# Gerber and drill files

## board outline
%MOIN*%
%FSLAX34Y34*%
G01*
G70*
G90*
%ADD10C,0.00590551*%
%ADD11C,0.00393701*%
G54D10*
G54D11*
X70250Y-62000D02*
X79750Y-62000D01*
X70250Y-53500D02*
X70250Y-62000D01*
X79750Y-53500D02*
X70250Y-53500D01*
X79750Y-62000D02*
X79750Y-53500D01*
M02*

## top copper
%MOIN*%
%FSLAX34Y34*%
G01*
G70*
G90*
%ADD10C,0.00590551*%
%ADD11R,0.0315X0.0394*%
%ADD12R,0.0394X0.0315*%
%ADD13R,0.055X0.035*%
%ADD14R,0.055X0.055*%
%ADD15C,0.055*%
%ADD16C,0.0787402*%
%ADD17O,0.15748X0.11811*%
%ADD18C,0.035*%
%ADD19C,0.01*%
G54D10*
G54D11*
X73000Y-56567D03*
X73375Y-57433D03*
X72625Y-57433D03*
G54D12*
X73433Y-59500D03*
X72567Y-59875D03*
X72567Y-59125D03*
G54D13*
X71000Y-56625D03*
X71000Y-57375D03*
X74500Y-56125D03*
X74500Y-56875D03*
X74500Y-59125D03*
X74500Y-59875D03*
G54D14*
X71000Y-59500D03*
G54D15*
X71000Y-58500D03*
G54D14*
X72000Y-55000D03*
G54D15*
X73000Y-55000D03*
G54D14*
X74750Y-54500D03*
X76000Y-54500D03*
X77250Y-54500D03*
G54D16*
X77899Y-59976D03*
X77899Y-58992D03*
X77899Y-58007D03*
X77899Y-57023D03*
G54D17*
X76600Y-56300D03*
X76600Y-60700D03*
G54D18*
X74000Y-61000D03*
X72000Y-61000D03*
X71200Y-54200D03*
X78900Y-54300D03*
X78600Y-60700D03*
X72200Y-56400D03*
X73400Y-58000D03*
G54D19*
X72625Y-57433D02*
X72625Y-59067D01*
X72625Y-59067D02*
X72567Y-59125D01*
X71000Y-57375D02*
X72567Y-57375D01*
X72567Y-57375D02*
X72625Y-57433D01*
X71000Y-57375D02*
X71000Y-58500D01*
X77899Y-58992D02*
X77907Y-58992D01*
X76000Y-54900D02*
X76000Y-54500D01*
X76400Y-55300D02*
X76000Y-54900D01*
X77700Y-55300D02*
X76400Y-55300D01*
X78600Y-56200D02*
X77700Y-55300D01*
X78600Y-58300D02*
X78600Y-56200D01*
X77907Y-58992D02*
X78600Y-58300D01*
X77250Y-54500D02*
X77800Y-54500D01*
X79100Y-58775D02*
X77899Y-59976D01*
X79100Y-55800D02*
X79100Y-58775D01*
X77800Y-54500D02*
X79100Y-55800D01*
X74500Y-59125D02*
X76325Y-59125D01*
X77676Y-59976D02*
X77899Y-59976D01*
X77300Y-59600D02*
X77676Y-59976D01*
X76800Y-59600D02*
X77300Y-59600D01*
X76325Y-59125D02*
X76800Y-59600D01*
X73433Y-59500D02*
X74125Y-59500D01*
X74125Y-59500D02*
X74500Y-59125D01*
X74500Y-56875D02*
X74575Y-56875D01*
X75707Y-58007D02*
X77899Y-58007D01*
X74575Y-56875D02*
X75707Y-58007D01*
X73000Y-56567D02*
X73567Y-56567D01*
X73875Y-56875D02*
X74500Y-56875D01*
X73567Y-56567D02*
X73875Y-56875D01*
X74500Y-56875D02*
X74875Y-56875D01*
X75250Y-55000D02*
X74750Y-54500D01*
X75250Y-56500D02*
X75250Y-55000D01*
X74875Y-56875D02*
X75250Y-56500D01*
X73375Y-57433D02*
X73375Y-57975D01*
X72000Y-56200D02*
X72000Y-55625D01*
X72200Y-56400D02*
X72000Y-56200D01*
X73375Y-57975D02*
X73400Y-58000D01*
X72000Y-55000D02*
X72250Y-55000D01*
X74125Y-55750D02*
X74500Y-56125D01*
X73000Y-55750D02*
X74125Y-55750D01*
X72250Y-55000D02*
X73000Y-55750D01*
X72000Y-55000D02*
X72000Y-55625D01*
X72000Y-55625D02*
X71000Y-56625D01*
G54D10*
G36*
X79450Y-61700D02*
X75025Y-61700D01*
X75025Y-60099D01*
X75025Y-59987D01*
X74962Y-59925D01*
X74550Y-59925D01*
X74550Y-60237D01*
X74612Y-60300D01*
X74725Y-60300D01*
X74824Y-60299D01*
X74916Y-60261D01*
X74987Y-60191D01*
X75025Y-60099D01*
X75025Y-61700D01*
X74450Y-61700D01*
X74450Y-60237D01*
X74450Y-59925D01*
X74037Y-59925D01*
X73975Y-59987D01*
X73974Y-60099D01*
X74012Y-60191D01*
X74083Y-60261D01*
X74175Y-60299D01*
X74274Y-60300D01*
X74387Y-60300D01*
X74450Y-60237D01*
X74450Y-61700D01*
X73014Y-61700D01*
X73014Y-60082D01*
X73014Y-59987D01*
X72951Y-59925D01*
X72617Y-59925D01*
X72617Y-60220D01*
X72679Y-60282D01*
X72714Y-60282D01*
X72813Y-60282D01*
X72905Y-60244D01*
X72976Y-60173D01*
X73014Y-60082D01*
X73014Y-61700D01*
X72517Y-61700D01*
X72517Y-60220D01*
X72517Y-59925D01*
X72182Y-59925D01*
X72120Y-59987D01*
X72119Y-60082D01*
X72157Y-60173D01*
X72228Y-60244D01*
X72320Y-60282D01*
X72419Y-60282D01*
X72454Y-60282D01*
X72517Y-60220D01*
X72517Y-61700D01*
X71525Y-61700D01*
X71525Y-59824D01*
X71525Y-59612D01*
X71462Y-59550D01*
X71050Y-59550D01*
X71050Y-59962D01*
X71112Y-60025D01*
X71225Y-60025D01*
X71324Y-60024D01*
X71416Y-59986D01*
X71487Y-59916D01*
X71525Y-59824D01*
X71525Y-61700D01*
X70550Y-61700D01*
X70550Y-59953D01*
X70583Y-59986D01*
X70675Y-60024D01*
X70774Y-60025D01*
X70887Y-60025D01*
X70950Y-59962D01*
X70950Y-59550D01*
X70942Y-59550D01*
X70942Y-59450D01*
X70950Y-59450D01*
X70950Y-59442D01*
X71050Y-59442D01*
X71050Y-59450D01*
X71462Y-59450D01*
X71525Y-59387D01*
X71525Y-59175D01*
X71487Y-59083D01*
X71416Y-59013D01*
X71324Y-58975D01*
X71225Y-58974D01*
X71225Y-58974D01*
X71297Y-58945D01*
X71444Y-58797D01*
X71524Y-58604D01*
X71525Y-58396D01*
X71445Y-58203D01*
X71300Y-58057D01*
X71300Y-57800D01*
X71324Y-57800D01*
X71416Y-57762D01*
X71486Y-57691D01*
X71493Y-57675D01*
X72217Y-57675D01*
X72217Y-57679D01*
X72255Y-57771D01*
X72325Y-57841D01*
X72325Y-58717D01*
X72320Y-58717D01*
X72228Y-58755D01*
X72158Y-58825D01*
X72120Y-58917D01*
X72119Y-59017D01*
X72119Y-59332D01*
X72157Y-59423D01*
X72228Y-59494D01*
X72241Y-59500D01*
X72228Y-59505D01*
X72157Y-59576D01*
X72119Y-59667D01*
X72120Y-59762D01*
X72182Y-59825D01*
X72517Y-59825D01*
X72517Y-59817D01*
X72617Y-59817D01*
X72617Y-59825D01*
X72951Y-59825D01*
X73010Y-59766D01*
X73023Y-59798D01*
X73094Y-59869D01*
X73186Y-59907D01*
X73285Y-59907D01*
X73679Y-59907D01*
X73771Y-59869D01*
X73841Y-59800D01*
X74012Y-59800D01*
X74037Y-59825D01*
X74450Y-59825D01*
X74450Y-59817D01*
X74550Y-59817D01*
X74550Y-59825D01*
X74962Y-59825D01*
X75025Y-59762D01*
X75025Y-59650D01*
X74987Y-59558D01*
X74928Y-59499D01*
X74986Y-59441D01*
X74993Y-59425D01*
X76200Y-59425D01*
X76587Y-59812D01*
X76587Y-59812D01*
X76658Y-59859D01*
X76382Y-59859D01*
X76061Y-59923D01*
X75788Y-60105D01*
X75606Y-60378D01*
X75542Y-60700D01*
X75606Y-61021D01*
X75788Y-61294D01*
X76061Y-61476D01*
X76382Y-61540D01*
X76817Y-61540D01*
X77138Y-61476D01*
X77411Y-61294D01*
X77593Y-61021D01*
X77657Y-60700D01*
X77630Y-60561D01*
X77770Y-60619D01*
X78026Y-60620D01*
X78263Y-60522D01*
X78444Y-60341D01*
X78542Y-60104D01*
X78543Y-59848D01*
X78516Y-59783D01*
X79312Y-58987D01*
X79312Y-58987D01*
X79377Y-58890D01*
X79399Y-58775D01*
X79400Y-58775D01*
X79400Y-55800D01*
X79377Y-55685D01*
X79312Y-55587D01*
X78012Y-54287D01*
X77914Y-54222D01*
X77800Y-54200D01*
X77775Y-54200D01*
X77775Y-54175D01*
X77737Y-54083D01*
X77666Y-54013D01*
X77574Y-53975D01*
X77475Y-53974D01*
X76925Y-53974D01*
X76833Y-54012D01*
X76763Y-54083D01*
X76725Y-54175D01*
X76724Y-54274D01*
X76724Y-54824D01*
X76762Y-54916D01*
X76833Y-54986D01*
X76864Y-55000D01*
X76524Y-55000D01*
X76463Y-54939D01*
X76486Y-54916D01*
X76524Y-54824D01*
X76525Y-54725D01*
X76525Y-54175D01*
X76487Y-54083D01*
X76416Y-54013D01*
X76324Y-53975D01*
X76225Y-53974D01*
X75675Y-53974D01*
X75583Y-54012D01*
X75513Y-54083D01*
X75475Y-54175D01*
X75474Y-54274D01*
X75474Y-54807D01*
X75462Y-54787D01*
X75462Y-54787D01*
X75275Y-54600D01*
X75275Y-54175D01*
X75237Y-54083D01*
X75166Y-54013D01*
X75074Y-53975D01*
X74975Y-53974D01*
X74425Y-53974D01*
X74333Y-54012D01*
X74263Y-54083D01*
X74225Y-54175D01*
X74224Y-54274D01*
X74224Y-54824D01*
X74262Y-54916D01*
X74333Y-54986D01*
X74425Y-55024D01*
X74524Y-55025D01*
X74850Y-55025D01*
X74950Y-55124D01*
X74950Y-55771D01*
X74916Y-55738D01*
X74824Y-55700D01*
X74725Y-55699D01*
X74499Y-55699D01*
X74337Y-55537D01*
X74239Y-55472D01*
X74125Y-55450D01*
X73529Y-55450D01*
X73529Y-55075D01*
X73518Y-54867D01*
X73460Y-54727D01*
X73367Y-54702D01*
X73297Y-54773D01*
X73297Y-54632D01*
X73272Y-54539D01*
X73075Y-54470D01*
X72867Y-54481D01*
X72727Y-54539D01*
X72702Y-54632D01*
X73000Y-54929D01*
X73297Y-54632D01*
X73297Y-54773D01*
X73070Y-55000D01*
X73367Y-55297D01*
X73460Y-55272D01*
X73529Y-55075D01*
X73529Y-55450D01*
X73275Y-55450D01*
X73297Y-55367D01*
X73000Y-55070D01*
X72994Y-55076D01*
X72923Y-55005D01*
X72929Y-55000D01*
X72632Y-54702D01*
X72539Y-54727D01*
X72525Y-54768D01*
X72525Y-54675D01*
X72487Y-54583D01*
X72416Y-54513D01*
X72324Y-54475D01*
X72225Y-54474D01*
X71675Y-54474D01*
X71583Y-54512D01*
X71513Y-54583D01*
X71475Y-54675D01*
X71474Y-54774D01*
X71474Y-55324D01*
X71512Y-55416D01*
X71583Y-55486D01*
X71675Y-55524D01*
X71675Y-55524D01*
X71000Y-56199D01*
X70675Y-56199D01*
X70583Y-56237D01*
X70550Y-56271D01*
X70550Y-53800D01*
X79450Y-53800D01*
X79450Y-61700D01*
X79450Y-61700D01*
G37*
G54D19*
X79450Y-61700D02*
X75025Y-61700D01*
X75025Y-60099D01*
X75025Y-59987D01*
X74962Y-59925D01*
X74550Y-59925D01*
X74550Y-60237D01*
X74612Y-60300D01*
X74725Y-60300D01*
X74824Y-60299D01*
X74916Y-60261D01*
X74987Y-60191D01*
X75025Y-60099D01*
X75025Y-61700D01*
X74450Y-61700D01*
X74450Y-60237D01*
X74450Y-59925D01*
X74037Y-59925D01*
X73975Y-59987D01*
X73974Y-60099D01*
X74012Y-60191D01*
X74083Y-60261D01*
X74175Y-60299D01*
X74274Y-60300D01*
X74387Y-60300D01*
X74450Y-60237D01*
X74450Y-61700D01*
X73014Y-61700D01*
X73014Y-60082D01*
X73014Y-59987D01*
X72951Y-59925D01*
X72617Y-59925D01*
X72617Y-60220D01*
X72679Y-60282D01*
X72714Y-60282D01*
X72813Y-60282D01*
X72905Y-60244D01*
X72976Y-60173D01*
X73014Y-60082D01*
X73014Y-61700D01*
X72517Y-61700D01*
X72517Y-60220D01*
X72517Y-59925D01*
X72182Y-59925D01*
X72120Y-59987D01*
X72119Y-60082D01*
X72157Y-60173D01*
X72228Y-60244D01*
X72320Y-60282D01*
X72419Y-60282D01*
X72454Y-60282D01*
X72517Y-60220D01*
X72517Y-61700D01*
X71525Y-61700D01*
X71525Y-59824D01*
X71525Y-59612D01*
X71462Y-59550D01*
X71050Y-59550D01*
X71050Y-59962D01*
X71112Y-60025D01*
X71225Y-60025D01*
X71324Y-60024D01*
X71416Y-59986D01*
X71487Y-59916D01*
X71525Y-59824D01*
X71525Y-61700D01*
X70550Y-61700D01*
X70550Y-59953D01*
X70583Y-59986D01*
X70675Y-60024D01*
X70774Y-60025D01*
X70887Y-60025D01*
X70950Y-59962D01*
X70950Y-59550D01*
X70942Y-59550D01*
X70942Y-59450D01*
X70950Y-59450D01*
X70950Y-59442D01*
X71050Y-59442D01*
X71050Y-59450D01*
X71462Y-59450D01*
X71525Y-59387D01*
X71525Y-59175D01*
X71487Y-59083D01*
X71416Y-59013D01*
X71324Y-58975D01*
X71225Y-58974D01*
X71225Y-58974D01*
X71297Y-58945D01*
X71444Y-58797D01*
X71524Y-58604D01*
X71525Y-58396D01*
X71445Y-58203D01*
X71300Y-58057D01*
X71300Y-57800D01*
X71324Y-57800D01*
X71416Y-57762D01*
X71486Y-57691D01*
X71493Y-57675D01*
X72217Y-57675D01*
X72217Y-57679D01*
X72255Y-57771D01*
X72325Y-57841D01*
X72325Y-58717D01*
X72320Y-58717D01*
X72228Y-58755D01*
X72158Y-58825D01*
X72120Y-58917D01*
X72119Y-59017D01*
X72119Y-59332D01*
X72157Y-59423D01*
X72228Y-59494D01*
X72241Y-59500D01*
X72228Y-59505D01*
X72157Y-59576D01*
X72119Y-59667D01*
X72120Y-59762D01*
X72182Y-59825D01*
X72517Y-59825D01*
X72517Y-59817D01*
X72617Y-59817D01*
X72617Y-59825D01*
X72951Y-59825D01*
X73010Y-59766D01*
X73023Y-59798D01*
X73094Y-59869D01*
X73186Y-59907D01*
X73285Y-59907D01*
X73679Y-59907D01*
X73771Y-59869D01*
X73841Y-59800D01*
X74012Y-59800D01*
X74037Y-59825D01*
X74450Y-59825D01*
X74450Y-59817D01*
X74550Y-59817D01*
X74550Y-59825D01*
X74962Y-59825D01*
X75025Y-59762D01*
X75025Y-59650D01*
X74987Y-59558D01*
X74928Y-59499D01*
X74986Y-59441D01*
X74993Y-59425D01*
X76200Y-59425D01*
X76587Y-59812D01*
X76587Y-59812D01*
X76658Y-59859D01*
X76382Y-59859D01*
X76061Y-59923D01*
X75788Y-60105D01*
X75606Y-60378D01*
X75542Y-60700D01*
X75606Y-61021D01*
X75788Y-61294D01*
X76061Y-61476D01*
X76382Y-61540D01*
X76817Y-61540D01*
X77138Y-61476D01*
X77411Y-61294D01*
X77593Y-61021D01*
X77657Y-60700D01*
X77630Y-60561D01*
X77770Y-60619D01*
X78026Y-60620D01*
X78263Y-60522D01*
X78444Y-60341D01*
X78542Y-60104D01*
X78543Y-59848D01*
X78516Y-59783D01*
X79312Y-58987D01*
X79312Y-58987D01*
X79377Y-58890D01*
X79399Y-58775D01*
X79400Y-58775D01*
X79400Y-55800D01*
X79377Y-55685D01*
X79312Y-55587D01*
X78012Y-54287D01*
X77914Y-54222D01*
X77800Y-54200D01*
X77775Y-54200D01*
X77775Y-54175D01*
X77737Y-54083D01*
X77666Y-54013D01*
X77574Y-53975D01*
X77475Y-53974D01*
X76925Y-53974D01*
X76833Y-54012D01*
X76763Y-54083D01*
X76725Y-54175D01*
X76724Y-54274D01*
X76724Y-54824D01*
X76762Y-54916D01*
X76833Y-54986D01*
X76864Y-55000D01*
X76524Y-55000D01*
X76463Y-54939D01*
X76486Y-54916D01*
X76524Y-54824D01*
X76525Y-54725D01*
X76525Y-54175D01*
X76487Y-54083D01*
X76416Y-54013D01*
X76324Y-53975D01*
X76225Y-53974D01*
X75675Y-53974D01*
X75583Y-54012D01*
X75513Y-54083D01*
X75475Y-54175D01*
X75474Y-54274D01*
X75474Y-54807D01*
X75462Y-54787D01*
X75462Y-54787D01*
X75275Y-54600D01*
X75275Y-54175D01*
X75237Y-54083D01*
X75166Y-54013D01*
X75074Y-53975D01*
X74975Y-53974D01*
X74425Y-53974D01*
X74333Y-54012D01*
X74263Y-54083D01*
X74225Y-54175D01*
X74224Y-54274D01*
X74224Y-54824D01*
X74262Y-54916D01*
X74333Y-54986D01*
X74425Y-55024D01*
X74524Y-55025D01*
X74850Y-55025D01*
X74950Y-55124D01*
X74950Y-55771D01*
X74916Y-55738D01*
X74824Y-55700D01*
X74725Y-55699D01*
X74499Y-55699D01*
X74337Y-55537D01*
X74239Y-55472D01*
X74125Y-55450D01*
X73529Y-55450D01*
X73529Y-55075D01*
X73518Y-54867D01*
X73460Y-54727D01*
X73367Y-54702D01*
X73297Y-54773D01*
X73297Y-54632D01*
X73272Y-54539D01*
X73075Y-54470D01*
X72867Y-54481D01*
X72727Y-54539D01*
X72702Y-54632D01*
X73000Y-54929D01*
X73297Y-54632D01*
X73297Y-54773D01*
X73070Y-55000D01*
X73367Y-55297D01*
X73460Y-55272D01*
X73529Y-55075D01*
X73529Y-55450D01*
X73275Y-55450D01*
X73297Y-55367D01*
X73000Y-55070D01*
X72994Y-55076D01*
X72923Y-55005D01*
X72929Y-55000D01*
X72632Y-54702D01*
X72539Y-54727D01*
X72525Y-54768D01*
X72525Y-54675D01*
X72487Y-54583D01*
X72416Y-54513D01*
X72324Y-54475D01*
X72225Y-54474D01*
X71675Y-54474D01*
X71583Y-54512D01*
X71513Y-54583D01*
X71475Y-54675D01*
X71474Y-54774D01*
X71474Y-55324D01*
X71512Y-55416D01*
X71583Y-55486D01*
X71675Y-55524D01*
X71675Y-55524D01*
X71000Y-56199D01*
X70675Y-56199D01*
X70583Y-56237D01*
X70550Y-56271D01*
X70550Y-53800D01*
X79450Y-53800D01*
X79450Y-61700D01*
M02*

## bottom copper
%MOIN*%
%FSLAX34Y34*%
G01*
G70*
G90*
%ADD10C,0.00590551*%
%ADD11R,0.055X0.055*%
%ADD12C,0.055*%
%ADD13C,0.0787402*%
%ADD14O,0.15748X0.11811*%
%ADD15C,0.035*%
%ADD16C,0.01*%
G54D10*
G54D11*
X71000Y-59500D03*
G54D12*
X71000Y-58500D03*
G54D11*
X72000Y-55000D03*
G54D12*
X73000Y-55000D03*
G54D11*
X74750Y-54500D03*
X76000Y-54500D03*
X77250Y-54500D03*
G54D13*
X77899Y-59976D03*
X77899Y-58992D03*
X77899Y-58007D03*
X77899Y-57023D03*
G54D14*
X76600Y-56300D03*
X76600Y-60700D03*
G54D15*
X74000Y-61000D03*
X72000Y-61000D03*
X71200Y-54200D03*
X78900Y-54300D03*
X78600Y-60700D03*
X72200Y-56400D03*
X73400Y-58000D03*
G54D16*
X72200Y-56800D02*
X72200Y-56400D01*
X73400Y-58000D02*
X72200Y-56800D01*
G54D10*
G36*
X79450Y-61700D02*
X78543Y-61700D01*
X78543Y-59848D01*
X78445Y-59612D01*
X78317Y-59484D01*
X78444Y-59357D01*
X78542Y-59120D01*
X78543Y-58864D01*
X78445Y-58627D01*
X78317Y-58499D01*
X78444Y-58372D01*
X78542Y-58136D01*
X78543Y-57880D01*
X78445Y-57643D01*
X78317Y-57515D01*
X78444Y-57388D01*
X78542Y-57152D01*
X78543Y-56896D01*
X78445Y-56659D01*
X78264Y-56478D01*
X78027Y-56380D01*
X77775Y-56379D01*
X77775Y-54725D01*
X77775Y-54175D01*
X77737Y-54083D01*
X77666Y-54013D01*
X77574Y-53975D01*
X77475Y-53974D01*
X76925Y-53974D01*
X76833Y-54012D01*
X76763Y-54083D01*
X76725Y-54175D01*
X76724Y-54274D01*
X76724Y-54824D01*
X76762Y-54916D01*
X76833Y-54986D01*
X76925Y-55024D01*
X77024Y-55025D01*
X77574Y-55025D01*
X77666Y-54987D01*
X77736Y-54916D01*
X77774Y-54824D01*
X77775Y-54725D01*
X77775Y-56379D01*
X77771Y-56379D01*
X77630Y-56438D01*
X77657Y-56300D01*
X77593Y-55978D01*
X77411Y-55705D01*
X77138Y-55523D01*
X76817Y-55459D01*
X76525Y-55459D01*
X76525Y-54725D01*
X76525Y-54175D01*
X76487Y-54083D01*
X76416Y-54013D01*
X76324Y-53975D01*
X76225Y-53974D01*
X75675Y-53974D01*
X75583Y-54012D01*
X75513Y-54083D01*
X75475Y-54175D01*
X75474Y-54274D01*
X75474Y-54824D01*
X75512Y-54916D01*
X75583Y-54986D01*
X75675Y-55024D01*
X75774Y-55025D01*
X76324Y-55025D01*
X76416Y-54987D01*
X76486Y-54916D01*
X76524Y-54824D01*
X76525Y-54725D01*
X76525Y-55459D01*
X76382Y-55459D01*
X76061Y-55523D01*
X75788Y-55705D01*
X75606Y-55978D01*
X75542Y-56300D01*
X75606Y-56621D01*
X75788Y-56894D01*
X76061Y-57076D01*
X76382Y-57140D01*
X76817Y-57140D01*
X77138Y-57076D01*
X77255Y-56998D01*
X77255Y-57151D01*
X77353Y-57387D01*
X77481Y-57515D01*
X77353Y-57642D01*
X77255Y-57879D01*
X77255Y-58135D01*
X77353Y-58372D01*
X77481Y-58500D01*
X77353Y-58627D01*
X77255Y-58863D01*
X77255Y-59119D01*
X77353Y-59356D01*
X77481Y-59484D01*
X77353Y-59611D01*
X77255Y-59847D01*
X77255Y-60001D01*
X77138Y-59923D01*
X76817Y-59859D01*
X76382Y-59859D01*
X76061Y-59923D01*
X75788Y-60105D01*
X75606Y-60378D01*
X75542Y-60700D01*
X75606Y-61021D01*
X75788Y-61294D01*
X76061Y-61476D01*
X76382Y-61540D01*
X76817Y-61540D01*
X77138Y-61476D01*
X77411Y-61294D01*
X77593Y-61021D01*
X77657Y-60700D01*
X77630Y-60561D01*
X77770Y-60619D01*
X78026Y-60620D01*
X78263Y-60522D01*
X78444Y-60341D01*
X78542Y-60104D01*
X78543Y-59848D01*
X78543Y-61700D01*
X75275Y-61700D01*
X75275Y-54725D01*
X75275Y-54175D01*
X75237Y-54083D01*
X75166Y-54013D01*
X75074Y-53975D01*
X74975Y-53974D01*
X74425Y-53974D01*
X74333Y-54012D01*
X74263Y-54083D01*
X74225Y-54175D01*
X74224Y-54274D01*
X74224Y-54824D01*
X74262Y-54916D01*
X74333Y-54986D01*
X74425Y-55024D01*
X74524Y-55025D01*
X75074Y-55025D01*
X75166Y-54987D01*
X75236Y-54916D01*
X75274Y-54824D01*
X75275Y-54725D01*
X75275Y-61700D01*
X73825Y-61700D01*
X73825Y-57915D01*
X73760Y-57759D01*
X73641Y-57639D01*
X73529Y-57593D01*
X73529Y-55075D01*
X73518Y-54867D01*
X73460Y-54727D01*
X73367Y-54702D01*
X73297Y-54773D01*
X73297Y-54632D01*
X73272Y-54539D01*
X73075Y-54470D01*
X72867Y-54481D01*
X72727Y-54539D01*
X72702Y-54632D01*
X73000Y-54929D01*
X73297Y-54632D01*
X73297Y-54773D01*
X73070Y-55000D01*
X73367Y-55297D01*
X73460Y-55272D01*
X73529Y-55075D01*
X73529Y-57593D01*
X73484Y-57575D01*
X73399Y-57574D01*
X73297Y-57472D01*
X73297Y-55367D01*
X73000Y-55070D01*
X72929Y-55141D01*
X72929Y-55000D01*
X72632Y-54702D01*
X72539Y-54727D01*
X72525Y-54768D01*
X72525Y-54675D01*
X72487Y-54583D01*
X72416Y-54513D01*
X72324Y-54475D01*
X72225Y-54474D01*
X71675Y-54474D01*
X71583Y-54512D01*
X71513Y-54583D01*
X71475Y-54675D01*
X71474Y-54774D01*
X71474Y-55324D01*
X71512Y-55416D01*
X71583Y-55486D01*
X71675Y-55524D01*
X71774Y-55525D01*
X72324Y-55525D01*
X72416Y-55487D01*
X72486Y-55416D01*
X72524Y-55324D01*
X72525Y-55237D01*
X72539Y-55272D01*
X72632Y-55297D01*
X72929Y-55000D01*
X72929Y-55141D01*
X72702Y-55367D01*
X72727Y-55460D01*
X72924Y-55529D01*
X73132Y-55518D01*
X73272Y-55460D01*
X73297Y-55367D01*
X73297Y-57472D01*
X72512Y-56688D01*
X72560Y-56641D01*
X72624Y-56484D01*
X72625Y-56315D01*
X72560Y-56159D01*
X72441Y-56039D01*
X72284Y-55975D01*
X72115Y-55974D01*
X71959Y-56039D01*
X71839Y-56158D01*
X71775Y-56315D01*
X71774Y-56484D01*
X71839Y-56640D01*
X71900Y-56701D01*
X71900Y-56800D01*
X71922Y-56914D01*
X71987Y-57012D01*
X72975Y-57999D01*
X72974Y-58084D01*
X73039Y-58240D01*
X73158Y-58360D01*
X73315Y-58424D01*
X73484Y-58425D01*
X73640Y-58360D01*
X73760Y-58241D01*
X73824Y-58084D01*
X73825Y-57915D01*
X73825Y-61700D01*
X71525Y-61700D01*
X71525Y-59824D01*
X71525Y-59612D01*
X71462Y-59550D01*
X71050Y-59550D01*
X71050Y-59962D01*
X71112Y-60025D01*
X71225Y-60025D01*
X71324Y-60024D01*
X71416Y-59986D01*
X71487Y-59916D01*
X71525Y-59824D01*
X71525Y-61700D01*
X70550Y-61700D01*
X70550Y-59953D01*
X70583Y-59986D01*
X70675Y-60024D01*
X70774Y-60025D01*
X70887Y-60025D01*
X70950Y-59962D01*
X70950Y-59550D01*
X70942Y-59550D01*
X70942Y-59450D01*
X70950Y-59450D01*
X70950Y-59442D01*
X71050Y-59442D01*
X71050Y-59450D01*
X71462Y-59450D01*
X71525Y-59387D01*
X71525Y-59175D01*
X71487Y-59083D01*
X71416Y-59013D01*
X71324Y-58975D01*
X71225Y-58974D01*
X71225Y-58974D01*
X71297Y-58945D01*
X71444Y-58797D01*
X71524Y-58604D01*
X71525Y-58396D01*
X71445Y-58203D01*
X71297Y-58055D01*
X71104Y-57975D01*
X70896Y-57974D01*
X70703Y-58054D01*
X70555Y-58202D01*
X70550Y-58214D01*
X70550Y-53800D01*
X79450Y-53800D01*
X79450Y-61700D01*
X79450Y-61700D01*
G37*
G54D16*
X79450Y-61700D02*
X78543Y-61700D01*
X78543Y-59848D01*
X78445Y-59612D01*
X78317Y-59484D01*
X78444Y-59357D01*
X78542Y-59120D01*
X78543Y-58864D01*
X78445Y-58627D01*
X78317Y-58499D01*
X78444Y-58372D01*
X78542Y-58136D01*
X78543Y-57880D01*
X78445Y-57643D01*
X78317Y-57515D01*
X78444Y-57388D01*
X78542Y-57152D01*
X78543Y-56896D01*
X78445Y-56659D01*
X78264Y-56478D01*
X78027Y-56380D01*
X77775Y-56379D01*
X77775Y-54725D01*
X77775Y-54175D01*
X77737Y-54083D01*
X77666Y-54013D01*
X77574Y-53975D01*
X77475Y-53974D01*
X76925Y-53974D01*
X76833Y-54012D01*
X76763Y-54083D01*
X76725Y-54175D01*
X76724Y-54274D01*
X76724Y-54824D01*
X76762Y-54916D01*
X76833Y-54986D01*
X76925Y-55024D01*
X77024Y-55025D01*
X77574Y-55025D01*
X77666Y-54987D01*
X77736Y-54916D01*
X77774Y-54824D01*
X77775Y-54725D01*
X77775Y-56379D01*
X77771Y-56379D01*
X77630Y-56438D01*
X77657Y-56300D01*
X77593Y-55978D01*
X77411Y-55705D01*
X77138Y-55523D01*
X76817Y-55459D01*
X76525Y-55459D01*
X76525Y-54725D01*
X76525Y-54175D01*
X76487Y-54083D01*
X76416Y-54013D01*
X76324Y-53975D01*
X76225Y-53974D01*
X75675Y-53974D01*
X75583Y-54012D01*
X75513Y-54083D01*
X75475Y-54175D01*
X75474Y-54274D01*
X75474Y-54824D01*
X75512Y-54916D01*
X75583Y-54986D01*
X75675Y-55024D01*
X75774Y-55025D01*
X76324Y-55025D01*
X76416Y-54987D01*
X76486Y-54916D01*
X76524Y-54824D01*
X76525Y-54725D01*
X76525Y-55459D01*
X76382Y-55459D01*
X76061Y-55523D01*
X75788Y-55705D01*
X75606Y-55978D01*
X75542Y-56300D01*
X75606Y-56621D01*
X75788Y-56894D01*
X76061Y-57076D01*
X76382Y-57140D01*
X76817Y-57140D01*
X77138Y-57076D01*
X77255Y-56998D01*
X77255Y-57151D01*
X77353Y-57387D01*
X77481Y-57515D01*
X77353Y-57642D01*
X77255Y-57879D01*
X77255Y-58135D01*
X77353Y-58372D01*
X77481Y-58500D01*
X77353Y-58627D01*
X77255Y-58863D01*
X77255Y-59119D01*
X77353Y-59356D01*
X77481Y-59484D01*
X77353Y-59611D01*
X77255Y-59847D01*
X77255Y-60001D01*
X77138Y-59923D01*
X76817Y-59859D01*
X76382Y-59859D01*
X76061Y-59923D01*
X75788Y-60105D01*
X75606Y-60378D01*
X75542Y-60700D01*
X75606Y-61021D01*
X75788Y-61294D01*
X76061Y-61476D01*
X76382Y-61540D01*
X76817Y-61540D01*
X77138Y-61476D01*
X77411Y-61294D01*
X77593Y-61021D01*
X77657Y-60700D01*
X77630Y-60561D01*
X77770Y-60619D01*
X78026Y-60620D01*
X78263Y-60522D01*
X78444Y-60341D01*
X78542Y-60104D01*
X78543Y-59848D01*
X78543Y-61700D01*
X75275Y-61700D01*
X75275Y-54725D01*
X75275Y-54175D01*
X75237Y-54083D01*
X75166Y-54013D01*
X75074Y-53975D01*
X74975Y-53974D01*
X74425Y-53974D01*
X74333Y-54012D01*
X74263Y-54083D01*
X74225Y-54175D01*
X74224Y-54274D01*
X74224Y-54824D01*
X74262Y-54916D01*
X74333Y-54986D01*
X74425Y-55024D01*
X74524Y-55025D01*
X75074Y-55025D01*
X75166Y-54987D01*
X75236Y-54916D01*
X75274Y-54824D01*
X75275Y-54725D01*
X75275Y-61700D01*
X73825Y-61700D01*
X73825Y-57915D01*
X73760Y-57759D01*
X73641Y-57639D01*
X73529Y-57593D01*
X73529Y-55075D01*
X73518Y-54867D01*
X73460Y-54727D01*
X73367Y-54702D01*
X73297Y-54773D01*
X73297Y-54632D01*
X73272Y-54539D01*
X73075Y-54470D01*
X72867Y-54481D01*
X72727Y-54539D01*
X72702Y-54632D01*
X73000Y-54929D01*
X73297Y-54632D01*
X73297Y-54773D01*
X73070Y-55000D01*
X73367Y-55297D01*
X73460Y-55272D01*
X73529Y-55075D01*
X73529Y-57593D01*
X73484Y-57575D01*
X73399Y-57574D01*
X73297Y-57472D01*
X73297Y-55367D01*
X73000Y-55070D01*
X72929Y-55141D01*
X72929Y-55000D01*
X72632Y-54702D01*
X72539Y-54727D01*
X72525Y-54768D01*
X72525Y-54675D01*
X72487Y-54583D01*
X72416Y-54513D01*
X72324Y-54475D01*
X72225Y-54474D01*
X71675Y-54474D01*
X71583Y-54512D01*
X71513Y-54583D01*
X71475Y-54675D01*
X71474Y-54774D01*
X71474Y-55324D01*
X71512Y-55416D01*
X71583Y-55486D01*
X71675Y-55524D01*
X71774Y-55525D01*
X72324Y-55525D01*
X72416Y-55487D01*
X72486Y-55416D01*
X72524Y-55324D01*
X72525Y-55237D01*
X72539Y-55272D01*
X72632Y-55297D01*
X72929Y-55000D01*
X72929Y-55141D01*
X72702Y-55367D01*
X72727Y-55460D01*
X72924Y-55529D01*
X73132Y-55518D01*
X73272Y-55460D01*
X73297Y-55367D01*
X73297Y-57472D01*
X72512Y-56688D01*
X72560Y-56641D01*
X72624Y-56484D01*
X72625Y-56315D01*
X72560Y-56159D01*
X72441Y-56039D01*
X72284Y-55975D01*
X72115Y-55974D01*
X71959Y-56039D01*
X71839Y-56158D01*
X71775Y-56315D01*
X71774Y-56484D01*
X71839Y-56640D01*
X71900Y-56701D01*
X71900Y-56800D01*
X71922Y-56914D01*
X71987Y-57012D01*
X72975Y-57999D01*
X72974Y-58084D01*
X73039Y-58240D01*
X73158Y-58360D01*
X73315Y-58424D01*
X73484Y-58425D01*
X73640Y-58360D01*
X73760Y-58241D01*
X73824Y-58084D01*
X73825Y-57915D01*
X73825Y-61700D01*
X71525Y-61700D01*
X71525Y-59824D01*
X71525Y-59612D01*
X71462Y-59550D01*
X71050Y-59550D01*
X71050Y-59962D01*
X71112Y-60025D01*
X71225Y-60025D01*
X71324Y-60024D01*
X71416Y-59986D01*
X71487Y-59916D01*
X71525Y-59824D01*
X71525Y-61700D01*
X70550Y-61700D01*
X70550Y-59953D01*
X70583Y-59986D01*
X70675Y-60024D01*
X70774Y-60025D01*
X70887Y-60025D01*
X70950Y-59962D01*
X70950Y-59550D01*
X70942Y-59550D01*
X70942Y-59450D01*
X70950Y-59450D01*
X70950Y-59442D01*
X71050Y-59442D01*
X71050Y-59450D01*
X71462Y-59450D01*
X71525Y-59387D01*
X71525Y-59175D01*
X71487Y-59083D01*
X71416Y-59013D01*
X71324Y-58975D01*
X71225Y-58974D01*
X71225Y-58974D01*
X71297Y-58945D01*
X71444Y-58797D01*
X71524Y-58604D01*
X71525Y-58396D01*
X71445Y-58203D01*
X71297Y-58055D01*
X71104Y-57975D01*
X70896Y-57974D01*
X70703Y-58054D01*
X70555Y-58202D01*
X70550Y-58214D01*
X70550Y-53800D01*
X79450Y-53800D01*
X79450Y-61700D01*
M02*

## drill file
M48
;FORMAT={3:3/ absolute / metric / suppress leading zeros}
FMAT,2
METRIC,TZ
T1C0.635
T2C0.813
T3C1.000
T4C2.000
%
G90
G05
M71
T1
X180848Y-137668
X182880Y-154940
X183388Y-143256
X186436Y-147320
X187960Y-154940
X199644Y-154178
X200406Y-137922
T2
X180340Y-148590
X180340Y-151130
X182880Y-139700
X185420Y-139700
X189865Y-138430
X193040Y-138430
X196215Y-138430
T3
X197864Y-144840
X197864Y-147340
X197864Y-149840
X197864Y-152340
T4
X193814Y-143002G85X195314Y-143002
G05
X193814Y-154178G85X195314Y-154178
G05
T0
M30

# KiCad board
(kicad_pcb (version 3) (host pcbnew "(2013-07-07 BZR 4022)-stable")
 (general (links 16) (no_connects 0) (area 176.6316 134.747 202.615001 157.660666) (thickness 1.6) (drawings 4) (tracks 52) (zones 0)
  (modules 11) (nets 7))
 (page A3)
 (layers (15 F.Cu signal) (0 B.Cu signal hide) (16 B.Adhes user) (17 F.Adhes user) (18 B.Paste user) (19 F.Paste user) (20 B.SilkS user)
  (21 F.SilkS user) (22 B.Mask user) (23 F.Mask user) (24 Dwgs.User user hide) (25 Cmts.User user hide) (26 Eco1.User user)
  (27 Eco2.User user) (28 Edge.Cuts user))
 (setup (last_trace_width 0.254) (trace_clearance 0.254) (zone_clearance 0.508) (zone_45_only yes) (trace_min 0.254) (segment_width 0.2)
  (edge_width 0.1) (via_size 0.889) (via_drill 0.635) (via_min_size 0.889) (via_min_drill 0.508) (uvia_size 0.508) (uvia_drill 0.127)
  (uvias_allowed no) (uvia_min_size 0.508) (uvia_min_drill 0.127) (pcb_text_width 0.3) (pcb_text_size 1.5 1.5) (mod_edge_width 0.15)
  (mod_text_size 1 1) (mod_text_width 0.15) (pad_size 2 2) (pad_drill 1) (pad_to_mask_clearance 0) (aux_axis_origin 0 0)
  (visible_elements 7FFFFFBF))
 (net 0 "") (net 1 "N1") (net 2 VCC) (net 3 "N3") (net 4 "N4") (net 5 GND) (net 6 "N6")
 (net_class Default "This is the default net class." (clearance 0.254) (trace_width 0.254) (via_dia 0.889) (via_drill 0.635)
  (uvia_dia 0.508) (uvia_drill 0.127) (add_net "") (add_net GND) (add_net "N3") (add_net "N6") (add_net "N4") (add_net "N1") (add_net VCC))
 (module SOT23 (layer F.Cu) (at 185.42 144.78)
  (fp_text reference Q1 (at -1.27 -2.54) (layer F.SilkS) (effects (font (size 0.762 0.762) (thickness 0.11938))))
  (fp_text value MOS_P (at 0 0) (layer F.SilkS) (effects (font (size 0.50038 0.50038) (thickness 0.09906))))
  (pad D smd rect (at 0 -1.09982) (size 0.8001 1.00076) (layers F.Cu F.Paste F.Mask) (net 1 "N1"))
  (pad S smd rect (at 0.9525 1.09982) (size 0.8001 1.00076) (layers F.Cu F.Paste F.Mask) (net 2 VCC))
  (pad G smd rect (at -0.9525 1.09982) (size 0.8001 1.00076) (layers F.Cu F.Paste F.Mask) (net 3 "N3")))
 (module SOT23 (layer F.Cu) (at 185.42 151.13 270)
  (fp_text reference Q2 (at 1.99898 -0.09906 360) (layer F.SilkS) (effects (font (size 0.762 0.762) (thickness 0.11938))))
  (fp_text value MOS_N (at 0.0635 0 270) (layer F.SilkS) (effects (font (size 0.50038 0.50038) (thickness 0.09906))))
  (pad D smd rect (at 0 -1.09982 270) (size 0.8001 1.00076) (layers F.Cu F.Paste F.Mask) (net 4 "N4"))
  (pad S smd rect (at 0.9525 1.09982 270) (size 0.8001 1.00076) (layers F.Cu F.Paste F.Mask) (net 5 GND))
  (pad G smd rect (at -0.9525 1.09982 270) (size 0.8001 1.00076) (layers F.Cu F.Paste F.Mask) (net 3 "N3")))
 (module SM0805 (layer F.Cu) (at 180.34 144.78 270)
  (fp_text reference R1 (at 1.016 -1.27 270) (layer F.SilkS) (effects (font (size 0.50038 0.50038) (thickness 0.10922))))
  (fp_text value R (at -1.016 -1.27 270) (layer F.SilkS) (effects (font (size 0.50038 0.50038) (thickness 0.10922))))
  (pad 1 smd rect (at -0.9525 0 270) (size 0.889 1.397) (layers F.Cu F.Paste F.Mask) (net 2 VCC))
  (pad 2 smd rect (at 0.9525 0 270) (size 0.889 1.397) (layers F.Cu F.Paste F.Mask) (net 3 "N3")))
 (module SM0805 (layer F.Cu) (at 189.23 143.51 270)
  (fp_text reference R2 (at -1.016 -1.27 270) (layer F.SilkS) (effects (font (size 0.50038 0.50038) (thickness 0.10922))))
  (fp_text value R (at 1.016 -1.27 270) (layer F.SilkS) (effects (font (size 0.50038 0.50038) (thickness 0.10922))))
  (pad 1 smd rect (at -0.9525 0 270) (size 0.889 1.397) (layers F.Cu F.Paste F.Mask) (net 2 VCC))
  (pad 2 smd rect (at 0.9525 0 270) (size 0.889 1.397) (layers F.Cu F.Paste F.Mask) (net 1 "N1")))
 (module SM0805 (layer F.Cu) (at 189.23 151.13 270)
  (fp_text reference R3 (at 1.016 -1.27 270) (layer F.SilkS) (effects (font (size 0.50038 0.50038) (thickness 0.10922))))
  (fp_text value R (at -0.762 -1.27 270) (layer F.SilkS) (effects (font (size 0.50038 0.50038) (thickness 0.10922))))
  (pad 1 smd rect (at -0.9525 0 270) (size 0.889 1.397) (layers F.Cu F.Paste F.Mask) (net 4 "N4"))
  (pad 2 smd rect (at 0.9525 0 270) (size 0.889 1.397) (layers F.Cu F.Paste F.Mask) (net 5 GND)))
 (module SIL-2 (layer F.Cu) (at 180.34 149.86 90)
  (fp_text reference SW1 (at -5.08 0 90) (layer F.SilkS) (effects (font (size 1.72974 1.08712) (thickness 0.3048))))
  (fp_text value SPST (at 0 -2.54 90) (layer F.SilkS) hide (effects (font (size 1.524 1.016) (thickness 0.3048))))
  (pad 1 thru_hole rect (at -1.27 0 90) (size 1.397 1.397) (drill 0.8128) (layers *.Cu *.Mask F.SilkS) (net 5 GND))
  (pad 2 thru_hole circle (at 1.27 0 90) (size 1.397 1.397) (drill 0.8128) (layers *.Cu *.Mask F.SilkS) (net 3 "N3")))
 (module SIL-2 (layer F.Cu) (at 184.15 139.7)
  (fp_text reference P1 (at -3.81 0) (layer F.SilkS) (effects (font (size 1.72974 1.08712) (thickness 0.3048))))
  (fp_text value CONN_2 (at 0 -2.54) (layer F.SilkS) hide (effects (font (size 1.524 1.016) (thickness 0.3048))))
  (pad 1 thru_hole rect (at -1.27 0) (size 1.397 1.397) (drill 0.8128) (layers *.Cu *.Mask F.SilkS) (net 2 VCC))
  (pad 2 thru_hole circle (at 1.27 0) (size 1.397 1.397) (drill 0.8128) (layers *.Cu *.Mask F.SilkS) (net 5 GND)))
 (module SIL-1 (layer F.Cu) (at 189.865 138.43)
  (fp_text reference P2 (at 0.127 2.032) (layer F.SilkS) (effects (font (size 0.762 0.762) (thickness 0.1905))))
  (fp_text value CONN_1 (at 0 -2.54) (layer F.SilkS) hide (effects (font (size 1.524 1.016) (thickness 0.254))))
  (pad 1 thru_hole rect (at 0 0) (size 1.397 1.397) (drill 0.8128) (layers *.Cu *.Mask F.SilkS) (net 1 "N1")))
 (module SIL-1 (layer F.Cu) (at 193.04 138.43)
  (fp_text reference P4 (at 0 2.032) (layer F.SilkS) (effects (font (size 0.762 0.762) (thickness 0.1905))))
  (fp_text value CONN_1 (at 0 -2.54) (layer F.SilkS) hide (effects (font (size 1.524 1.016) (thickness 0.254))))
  (pad 1 thru_hole rect (at 0 0) (size 1.397 1.397) (drill 0.8128) (layers *.Cu *.Mask F.SilkS) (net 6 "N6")))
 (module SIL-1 (layer F.Cu) (at 196.215 138.43)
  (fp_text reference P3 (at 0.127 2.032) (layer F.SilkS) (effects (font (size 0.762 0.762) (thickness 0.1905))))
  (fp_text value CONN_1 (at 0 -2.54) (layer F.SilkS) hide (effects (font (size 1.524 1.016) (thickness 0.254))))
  (pad 1 thru_hole rect (at 0 0) (size 1.397 1.397) (drill 0.8128) (layers *.Cu *.Mask F.SilkS) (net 4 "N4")))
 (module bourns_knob (layer F.Cu) (at 194.564 148.59 90)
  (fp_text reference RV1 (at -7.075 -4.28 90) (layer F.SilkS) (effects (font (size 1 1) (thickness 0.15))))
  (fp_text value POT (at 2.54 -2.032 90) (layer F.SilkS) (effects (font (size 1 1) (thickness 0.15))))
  (pad 3 thru_hole circle (at -3.75 3.3 90) (size 2 2) (drill 1) (layers *.Cu *.Mask F.SilkS) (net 4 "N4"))
  (pad 2 thru_hole circle (at -1.25 3.3 90) (size 2 2) (drill 1) (layers *.Cu *.Mask F.SilkS) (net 6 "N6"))
  (pad 1 thru_hole circle (at 1.25 3.3 90) (size 2 2) (drill 1) (layers *.Cu *.Mask F.SilkS) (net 1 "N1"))
  (pad 4 thru_hole circle (at 3.75 3.3 90) (size 2 2) (drill 1) (layers *.Cu *.Mask F.SilkS))
  (pad "" thru_hole oval (at 5.588 0 90) (size 3 4) (drill oval 2 3.5) (layers *.Cu *.Mask F.SilkS))
  (pad "" thru_hole oval (at -5.588 0 90) (size 3 4) (drill oval 2 3.5) (layers *.Cu *.Mask F.SilkS)))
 (gr_line (start 178.435 157.48) (end 202.565 157.48) (angle 90) (layer Edge.Cuts) (width 0.1))
 (gr_line (start 178.435 135.89) (end 178.435 157.48) (angle 90) (layer Edge.Cuts) (width 0.1))
 (gr_line (start 202.565 135.89) (end 178.435 135.89) (angle 90) (layer Edge.Cuts) (width 0.1))
 (gr_line (start 202.565 157.48) (end 202.565 135.89) (angle 90) (layer Edge.Cuts) (width 0.1))
 (via (at 187.96 154.94) (size 0.889) (layers F.Cu B.Cu) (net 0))
 (via (at 182.88 154.94) (size 0.889) (layers F.Cu B.Cu) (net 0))
 (via (at 180.848 137.668) (size 0.889) (layers F.Cu B.Cu) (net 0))
 (via (at 200.406 137.922) (size 0.889) (layers F.Cu B.Cu) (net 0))
 (via (at 199.644 154.178) (size 0.889) (layers F.Cu B.Cu) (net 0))
 (segment (start 184.4675 145.87982) (end 184.4675 150.03018) (width 0.254) (layer F.Cu) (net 3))
 (segment (start 184.4675 150.03018) (end 184.32018 150.1775) (width 0.254) (layer F.Cu) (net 3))
 (segment (start 180.34 145.7325) (end 184.32018 145.7325) (width 0.254) (layer F.Cu) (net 3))
 (segment (start 184.32018 145.7325) (end 184.4675 145.87982) (width 0.254) (layer F.Cu) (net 3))
 (segment (start 180.34 145.7325) (end 180.34 148.59) (width 0.254) (layer F.Cu) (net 3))
 (segment (start 197.864 149.84) (end 197.886 149.84) (width 0.254) (layer F.Cu) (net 6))
 (segment (start 193.04 139.446) (end 193.04 138.43) (width 0.254) (layer F.Cu) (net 6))
 (segment (start 194.056 140.462) (end 193.04 139.446) (width 0.254) (layer F.Cu) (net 6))
 (segment (start 197.358 140.462) (end 194.056 140.462) (width 0.254) (layer F.Cu) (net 6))
 (segment (start 199.644 142.748) (end 197.358 140.462) (width 0.254) (layer F.Cu) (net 6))
 (segment (start 199.644 148.082) (end 199.644 142.748) (width 0.254) (layer F.Cu) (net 6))
 (segment (start 197.886 149.84) (end 199.644 148.082) (width 0.254) (layer F.Cu) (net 6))
 (segment (start 196.215 138.43) (end 197.612 138.43) (width 0.254) (layer F.Cu) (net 4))
 (segment (start 200.914 149.29) (end 197.864 152.34) (width 0.254) (layer F.Cu) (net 4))
 (segment (start 200.914 141.732) (end 200.914 149.29) (width 0.254) (layer F.Cu) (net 4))
 (segment (start 197.612 138.43) (end 200.914 141.732) (width 0.254) (layer F.Cu) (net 4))
 (segment (start 189.23 150.1775) (end 193.8655 150.1775) (width 0.254) (layer F.Cu) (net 4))
 (segment (start 197.298 152.34) (end 197.864 152.34) (width 0.254) (layer F.Cu) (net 4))
 (segment (start 196.342 151.384) (end 197.298 152.34) (width 0.254) (layer F.Cu) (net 4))
 (segment (start 195.072 151.384) (end 196.342 151.384) (width 0.254) (layer F.Cu) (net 4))
 (segment (start 193.8655 150.1775) (end 195.072 151.384) (width 0.254) (layer F.Cu) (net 4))
 (segment (start 186.51982 151.13) (end 188.2775 151.13) (width 0.254) (layer F.Cu) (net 4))
 (segment (start 188.2775 151.13) (end 189.23 150.1775) (width 0.254) (layer F.Cu) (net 4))
 (segment (start 189.23 144.4625) (end 189.4205 144.4625) (width 0.254) (layer F.Cu) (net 1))
 (segment (start 192.298 147.34) (end 197.864 147.34) (width 0.254) (layer F.Cu) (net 1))
 (segment (start 189.4205 144.4625) (end 192.298 147.34) (width 0.254) (layer F.Cu) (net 1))
 (segment (start 185.42 143.68018) (end 186.86018 143.68018) (width 0.254) (layer F.Cu) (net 1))
 (segment (start 187.6425 144.4625) (end 189.23 144.4625) (width 0.254) (layer F.Cu) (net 1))
 (segment (start 186.86018 143.68018) (end 187.6425 144.4625) (width 0.254) (layer F.Cu) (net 1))
 (segment (start 189.23 144.4625) (end 190.1825 144.4625) (width 0.254) (layer F.Cu) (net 1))
 (segment (start 191.135 139.7) (end 189.865 138.43) (width 0.254) (layer F.Cu) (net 1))
 (segment (start 191.135 143.51) (end 191.135 139.7) (width 0.254) (layer F.Cu) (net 1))
 (segment (start 190.1825 144.4625) (end 191.135 143.51) (width 0.254) (layer F.Cu) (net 1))
 (segment (start 186.3725 145.87982) (end 186.3725 147.2565) (width 0.254) (layer F.Cu) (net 2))
 (segment (start 182.88 142.748) (end 182.88 141.2875) (width 0.254) (layer F.Cu) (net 2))
 (segment (start 183.388 143.256) (end 182.88 142.748) (width 0.254) (layer F.Cu) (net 2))
 (via (at 183.388 143.256) (size 0.889) (layers F.Cu B.Cu) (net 2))
 (segment (start 183.388 144.272) (end 183.388 143.256) (width 0.254) (layer B.Cu) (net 2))
 (segment (start 186.436 147.32) (end 183.388 144.272) (width 0.254) (layer B.Cu) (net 2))
 (via (at 186.436 147.32) (size 0.889) (layers F.Cu B.Cu) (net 2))
 (segment (start 186.3725 147.2565) (end 186.436 147.32) (width 0.254) (layer F.Cu) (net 2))
 (segment (start 182.88 139.7) (end 183.515 139.7) (width 0.254) (layer F.Cu) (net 2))
 (segment (start 188.2775 141.605) (end 189.23 142.5575) (width 0.254) (layer F.Cu) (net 2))
 (segment (start 185.42 141.605) (end 188.2775 141.605) (width 0.254) (layer F.Cu) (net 2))
 (segment (start 183.515 139.7) (end 185.42 141.605) (width 0.254) (layer F.Cu) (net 2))
 (segment (start 182.88 139.7) (end 182.88 141.2875) (width 0.254) (layer F.Cu) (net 2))
 (segment (start 182.88 141.2875) (end 180.34 143.8275) (width 0.254) (layer F.Cu) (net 2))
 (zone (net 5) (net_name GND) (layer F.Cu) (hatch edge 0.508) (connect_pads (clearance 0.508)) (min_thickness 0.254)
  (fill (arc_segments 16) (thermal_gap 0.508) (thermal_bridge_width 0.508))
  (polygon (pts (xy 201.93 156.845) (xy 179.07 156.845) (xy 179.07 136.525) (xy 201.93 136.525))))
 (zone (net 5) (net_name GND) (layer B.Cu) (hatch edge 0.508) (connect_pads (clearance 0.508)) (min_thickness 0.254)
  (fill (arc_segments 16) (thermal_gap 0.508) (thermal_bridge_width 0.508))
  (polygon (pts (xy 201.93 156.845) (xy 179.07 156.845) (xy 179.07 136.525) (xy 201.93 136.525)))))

